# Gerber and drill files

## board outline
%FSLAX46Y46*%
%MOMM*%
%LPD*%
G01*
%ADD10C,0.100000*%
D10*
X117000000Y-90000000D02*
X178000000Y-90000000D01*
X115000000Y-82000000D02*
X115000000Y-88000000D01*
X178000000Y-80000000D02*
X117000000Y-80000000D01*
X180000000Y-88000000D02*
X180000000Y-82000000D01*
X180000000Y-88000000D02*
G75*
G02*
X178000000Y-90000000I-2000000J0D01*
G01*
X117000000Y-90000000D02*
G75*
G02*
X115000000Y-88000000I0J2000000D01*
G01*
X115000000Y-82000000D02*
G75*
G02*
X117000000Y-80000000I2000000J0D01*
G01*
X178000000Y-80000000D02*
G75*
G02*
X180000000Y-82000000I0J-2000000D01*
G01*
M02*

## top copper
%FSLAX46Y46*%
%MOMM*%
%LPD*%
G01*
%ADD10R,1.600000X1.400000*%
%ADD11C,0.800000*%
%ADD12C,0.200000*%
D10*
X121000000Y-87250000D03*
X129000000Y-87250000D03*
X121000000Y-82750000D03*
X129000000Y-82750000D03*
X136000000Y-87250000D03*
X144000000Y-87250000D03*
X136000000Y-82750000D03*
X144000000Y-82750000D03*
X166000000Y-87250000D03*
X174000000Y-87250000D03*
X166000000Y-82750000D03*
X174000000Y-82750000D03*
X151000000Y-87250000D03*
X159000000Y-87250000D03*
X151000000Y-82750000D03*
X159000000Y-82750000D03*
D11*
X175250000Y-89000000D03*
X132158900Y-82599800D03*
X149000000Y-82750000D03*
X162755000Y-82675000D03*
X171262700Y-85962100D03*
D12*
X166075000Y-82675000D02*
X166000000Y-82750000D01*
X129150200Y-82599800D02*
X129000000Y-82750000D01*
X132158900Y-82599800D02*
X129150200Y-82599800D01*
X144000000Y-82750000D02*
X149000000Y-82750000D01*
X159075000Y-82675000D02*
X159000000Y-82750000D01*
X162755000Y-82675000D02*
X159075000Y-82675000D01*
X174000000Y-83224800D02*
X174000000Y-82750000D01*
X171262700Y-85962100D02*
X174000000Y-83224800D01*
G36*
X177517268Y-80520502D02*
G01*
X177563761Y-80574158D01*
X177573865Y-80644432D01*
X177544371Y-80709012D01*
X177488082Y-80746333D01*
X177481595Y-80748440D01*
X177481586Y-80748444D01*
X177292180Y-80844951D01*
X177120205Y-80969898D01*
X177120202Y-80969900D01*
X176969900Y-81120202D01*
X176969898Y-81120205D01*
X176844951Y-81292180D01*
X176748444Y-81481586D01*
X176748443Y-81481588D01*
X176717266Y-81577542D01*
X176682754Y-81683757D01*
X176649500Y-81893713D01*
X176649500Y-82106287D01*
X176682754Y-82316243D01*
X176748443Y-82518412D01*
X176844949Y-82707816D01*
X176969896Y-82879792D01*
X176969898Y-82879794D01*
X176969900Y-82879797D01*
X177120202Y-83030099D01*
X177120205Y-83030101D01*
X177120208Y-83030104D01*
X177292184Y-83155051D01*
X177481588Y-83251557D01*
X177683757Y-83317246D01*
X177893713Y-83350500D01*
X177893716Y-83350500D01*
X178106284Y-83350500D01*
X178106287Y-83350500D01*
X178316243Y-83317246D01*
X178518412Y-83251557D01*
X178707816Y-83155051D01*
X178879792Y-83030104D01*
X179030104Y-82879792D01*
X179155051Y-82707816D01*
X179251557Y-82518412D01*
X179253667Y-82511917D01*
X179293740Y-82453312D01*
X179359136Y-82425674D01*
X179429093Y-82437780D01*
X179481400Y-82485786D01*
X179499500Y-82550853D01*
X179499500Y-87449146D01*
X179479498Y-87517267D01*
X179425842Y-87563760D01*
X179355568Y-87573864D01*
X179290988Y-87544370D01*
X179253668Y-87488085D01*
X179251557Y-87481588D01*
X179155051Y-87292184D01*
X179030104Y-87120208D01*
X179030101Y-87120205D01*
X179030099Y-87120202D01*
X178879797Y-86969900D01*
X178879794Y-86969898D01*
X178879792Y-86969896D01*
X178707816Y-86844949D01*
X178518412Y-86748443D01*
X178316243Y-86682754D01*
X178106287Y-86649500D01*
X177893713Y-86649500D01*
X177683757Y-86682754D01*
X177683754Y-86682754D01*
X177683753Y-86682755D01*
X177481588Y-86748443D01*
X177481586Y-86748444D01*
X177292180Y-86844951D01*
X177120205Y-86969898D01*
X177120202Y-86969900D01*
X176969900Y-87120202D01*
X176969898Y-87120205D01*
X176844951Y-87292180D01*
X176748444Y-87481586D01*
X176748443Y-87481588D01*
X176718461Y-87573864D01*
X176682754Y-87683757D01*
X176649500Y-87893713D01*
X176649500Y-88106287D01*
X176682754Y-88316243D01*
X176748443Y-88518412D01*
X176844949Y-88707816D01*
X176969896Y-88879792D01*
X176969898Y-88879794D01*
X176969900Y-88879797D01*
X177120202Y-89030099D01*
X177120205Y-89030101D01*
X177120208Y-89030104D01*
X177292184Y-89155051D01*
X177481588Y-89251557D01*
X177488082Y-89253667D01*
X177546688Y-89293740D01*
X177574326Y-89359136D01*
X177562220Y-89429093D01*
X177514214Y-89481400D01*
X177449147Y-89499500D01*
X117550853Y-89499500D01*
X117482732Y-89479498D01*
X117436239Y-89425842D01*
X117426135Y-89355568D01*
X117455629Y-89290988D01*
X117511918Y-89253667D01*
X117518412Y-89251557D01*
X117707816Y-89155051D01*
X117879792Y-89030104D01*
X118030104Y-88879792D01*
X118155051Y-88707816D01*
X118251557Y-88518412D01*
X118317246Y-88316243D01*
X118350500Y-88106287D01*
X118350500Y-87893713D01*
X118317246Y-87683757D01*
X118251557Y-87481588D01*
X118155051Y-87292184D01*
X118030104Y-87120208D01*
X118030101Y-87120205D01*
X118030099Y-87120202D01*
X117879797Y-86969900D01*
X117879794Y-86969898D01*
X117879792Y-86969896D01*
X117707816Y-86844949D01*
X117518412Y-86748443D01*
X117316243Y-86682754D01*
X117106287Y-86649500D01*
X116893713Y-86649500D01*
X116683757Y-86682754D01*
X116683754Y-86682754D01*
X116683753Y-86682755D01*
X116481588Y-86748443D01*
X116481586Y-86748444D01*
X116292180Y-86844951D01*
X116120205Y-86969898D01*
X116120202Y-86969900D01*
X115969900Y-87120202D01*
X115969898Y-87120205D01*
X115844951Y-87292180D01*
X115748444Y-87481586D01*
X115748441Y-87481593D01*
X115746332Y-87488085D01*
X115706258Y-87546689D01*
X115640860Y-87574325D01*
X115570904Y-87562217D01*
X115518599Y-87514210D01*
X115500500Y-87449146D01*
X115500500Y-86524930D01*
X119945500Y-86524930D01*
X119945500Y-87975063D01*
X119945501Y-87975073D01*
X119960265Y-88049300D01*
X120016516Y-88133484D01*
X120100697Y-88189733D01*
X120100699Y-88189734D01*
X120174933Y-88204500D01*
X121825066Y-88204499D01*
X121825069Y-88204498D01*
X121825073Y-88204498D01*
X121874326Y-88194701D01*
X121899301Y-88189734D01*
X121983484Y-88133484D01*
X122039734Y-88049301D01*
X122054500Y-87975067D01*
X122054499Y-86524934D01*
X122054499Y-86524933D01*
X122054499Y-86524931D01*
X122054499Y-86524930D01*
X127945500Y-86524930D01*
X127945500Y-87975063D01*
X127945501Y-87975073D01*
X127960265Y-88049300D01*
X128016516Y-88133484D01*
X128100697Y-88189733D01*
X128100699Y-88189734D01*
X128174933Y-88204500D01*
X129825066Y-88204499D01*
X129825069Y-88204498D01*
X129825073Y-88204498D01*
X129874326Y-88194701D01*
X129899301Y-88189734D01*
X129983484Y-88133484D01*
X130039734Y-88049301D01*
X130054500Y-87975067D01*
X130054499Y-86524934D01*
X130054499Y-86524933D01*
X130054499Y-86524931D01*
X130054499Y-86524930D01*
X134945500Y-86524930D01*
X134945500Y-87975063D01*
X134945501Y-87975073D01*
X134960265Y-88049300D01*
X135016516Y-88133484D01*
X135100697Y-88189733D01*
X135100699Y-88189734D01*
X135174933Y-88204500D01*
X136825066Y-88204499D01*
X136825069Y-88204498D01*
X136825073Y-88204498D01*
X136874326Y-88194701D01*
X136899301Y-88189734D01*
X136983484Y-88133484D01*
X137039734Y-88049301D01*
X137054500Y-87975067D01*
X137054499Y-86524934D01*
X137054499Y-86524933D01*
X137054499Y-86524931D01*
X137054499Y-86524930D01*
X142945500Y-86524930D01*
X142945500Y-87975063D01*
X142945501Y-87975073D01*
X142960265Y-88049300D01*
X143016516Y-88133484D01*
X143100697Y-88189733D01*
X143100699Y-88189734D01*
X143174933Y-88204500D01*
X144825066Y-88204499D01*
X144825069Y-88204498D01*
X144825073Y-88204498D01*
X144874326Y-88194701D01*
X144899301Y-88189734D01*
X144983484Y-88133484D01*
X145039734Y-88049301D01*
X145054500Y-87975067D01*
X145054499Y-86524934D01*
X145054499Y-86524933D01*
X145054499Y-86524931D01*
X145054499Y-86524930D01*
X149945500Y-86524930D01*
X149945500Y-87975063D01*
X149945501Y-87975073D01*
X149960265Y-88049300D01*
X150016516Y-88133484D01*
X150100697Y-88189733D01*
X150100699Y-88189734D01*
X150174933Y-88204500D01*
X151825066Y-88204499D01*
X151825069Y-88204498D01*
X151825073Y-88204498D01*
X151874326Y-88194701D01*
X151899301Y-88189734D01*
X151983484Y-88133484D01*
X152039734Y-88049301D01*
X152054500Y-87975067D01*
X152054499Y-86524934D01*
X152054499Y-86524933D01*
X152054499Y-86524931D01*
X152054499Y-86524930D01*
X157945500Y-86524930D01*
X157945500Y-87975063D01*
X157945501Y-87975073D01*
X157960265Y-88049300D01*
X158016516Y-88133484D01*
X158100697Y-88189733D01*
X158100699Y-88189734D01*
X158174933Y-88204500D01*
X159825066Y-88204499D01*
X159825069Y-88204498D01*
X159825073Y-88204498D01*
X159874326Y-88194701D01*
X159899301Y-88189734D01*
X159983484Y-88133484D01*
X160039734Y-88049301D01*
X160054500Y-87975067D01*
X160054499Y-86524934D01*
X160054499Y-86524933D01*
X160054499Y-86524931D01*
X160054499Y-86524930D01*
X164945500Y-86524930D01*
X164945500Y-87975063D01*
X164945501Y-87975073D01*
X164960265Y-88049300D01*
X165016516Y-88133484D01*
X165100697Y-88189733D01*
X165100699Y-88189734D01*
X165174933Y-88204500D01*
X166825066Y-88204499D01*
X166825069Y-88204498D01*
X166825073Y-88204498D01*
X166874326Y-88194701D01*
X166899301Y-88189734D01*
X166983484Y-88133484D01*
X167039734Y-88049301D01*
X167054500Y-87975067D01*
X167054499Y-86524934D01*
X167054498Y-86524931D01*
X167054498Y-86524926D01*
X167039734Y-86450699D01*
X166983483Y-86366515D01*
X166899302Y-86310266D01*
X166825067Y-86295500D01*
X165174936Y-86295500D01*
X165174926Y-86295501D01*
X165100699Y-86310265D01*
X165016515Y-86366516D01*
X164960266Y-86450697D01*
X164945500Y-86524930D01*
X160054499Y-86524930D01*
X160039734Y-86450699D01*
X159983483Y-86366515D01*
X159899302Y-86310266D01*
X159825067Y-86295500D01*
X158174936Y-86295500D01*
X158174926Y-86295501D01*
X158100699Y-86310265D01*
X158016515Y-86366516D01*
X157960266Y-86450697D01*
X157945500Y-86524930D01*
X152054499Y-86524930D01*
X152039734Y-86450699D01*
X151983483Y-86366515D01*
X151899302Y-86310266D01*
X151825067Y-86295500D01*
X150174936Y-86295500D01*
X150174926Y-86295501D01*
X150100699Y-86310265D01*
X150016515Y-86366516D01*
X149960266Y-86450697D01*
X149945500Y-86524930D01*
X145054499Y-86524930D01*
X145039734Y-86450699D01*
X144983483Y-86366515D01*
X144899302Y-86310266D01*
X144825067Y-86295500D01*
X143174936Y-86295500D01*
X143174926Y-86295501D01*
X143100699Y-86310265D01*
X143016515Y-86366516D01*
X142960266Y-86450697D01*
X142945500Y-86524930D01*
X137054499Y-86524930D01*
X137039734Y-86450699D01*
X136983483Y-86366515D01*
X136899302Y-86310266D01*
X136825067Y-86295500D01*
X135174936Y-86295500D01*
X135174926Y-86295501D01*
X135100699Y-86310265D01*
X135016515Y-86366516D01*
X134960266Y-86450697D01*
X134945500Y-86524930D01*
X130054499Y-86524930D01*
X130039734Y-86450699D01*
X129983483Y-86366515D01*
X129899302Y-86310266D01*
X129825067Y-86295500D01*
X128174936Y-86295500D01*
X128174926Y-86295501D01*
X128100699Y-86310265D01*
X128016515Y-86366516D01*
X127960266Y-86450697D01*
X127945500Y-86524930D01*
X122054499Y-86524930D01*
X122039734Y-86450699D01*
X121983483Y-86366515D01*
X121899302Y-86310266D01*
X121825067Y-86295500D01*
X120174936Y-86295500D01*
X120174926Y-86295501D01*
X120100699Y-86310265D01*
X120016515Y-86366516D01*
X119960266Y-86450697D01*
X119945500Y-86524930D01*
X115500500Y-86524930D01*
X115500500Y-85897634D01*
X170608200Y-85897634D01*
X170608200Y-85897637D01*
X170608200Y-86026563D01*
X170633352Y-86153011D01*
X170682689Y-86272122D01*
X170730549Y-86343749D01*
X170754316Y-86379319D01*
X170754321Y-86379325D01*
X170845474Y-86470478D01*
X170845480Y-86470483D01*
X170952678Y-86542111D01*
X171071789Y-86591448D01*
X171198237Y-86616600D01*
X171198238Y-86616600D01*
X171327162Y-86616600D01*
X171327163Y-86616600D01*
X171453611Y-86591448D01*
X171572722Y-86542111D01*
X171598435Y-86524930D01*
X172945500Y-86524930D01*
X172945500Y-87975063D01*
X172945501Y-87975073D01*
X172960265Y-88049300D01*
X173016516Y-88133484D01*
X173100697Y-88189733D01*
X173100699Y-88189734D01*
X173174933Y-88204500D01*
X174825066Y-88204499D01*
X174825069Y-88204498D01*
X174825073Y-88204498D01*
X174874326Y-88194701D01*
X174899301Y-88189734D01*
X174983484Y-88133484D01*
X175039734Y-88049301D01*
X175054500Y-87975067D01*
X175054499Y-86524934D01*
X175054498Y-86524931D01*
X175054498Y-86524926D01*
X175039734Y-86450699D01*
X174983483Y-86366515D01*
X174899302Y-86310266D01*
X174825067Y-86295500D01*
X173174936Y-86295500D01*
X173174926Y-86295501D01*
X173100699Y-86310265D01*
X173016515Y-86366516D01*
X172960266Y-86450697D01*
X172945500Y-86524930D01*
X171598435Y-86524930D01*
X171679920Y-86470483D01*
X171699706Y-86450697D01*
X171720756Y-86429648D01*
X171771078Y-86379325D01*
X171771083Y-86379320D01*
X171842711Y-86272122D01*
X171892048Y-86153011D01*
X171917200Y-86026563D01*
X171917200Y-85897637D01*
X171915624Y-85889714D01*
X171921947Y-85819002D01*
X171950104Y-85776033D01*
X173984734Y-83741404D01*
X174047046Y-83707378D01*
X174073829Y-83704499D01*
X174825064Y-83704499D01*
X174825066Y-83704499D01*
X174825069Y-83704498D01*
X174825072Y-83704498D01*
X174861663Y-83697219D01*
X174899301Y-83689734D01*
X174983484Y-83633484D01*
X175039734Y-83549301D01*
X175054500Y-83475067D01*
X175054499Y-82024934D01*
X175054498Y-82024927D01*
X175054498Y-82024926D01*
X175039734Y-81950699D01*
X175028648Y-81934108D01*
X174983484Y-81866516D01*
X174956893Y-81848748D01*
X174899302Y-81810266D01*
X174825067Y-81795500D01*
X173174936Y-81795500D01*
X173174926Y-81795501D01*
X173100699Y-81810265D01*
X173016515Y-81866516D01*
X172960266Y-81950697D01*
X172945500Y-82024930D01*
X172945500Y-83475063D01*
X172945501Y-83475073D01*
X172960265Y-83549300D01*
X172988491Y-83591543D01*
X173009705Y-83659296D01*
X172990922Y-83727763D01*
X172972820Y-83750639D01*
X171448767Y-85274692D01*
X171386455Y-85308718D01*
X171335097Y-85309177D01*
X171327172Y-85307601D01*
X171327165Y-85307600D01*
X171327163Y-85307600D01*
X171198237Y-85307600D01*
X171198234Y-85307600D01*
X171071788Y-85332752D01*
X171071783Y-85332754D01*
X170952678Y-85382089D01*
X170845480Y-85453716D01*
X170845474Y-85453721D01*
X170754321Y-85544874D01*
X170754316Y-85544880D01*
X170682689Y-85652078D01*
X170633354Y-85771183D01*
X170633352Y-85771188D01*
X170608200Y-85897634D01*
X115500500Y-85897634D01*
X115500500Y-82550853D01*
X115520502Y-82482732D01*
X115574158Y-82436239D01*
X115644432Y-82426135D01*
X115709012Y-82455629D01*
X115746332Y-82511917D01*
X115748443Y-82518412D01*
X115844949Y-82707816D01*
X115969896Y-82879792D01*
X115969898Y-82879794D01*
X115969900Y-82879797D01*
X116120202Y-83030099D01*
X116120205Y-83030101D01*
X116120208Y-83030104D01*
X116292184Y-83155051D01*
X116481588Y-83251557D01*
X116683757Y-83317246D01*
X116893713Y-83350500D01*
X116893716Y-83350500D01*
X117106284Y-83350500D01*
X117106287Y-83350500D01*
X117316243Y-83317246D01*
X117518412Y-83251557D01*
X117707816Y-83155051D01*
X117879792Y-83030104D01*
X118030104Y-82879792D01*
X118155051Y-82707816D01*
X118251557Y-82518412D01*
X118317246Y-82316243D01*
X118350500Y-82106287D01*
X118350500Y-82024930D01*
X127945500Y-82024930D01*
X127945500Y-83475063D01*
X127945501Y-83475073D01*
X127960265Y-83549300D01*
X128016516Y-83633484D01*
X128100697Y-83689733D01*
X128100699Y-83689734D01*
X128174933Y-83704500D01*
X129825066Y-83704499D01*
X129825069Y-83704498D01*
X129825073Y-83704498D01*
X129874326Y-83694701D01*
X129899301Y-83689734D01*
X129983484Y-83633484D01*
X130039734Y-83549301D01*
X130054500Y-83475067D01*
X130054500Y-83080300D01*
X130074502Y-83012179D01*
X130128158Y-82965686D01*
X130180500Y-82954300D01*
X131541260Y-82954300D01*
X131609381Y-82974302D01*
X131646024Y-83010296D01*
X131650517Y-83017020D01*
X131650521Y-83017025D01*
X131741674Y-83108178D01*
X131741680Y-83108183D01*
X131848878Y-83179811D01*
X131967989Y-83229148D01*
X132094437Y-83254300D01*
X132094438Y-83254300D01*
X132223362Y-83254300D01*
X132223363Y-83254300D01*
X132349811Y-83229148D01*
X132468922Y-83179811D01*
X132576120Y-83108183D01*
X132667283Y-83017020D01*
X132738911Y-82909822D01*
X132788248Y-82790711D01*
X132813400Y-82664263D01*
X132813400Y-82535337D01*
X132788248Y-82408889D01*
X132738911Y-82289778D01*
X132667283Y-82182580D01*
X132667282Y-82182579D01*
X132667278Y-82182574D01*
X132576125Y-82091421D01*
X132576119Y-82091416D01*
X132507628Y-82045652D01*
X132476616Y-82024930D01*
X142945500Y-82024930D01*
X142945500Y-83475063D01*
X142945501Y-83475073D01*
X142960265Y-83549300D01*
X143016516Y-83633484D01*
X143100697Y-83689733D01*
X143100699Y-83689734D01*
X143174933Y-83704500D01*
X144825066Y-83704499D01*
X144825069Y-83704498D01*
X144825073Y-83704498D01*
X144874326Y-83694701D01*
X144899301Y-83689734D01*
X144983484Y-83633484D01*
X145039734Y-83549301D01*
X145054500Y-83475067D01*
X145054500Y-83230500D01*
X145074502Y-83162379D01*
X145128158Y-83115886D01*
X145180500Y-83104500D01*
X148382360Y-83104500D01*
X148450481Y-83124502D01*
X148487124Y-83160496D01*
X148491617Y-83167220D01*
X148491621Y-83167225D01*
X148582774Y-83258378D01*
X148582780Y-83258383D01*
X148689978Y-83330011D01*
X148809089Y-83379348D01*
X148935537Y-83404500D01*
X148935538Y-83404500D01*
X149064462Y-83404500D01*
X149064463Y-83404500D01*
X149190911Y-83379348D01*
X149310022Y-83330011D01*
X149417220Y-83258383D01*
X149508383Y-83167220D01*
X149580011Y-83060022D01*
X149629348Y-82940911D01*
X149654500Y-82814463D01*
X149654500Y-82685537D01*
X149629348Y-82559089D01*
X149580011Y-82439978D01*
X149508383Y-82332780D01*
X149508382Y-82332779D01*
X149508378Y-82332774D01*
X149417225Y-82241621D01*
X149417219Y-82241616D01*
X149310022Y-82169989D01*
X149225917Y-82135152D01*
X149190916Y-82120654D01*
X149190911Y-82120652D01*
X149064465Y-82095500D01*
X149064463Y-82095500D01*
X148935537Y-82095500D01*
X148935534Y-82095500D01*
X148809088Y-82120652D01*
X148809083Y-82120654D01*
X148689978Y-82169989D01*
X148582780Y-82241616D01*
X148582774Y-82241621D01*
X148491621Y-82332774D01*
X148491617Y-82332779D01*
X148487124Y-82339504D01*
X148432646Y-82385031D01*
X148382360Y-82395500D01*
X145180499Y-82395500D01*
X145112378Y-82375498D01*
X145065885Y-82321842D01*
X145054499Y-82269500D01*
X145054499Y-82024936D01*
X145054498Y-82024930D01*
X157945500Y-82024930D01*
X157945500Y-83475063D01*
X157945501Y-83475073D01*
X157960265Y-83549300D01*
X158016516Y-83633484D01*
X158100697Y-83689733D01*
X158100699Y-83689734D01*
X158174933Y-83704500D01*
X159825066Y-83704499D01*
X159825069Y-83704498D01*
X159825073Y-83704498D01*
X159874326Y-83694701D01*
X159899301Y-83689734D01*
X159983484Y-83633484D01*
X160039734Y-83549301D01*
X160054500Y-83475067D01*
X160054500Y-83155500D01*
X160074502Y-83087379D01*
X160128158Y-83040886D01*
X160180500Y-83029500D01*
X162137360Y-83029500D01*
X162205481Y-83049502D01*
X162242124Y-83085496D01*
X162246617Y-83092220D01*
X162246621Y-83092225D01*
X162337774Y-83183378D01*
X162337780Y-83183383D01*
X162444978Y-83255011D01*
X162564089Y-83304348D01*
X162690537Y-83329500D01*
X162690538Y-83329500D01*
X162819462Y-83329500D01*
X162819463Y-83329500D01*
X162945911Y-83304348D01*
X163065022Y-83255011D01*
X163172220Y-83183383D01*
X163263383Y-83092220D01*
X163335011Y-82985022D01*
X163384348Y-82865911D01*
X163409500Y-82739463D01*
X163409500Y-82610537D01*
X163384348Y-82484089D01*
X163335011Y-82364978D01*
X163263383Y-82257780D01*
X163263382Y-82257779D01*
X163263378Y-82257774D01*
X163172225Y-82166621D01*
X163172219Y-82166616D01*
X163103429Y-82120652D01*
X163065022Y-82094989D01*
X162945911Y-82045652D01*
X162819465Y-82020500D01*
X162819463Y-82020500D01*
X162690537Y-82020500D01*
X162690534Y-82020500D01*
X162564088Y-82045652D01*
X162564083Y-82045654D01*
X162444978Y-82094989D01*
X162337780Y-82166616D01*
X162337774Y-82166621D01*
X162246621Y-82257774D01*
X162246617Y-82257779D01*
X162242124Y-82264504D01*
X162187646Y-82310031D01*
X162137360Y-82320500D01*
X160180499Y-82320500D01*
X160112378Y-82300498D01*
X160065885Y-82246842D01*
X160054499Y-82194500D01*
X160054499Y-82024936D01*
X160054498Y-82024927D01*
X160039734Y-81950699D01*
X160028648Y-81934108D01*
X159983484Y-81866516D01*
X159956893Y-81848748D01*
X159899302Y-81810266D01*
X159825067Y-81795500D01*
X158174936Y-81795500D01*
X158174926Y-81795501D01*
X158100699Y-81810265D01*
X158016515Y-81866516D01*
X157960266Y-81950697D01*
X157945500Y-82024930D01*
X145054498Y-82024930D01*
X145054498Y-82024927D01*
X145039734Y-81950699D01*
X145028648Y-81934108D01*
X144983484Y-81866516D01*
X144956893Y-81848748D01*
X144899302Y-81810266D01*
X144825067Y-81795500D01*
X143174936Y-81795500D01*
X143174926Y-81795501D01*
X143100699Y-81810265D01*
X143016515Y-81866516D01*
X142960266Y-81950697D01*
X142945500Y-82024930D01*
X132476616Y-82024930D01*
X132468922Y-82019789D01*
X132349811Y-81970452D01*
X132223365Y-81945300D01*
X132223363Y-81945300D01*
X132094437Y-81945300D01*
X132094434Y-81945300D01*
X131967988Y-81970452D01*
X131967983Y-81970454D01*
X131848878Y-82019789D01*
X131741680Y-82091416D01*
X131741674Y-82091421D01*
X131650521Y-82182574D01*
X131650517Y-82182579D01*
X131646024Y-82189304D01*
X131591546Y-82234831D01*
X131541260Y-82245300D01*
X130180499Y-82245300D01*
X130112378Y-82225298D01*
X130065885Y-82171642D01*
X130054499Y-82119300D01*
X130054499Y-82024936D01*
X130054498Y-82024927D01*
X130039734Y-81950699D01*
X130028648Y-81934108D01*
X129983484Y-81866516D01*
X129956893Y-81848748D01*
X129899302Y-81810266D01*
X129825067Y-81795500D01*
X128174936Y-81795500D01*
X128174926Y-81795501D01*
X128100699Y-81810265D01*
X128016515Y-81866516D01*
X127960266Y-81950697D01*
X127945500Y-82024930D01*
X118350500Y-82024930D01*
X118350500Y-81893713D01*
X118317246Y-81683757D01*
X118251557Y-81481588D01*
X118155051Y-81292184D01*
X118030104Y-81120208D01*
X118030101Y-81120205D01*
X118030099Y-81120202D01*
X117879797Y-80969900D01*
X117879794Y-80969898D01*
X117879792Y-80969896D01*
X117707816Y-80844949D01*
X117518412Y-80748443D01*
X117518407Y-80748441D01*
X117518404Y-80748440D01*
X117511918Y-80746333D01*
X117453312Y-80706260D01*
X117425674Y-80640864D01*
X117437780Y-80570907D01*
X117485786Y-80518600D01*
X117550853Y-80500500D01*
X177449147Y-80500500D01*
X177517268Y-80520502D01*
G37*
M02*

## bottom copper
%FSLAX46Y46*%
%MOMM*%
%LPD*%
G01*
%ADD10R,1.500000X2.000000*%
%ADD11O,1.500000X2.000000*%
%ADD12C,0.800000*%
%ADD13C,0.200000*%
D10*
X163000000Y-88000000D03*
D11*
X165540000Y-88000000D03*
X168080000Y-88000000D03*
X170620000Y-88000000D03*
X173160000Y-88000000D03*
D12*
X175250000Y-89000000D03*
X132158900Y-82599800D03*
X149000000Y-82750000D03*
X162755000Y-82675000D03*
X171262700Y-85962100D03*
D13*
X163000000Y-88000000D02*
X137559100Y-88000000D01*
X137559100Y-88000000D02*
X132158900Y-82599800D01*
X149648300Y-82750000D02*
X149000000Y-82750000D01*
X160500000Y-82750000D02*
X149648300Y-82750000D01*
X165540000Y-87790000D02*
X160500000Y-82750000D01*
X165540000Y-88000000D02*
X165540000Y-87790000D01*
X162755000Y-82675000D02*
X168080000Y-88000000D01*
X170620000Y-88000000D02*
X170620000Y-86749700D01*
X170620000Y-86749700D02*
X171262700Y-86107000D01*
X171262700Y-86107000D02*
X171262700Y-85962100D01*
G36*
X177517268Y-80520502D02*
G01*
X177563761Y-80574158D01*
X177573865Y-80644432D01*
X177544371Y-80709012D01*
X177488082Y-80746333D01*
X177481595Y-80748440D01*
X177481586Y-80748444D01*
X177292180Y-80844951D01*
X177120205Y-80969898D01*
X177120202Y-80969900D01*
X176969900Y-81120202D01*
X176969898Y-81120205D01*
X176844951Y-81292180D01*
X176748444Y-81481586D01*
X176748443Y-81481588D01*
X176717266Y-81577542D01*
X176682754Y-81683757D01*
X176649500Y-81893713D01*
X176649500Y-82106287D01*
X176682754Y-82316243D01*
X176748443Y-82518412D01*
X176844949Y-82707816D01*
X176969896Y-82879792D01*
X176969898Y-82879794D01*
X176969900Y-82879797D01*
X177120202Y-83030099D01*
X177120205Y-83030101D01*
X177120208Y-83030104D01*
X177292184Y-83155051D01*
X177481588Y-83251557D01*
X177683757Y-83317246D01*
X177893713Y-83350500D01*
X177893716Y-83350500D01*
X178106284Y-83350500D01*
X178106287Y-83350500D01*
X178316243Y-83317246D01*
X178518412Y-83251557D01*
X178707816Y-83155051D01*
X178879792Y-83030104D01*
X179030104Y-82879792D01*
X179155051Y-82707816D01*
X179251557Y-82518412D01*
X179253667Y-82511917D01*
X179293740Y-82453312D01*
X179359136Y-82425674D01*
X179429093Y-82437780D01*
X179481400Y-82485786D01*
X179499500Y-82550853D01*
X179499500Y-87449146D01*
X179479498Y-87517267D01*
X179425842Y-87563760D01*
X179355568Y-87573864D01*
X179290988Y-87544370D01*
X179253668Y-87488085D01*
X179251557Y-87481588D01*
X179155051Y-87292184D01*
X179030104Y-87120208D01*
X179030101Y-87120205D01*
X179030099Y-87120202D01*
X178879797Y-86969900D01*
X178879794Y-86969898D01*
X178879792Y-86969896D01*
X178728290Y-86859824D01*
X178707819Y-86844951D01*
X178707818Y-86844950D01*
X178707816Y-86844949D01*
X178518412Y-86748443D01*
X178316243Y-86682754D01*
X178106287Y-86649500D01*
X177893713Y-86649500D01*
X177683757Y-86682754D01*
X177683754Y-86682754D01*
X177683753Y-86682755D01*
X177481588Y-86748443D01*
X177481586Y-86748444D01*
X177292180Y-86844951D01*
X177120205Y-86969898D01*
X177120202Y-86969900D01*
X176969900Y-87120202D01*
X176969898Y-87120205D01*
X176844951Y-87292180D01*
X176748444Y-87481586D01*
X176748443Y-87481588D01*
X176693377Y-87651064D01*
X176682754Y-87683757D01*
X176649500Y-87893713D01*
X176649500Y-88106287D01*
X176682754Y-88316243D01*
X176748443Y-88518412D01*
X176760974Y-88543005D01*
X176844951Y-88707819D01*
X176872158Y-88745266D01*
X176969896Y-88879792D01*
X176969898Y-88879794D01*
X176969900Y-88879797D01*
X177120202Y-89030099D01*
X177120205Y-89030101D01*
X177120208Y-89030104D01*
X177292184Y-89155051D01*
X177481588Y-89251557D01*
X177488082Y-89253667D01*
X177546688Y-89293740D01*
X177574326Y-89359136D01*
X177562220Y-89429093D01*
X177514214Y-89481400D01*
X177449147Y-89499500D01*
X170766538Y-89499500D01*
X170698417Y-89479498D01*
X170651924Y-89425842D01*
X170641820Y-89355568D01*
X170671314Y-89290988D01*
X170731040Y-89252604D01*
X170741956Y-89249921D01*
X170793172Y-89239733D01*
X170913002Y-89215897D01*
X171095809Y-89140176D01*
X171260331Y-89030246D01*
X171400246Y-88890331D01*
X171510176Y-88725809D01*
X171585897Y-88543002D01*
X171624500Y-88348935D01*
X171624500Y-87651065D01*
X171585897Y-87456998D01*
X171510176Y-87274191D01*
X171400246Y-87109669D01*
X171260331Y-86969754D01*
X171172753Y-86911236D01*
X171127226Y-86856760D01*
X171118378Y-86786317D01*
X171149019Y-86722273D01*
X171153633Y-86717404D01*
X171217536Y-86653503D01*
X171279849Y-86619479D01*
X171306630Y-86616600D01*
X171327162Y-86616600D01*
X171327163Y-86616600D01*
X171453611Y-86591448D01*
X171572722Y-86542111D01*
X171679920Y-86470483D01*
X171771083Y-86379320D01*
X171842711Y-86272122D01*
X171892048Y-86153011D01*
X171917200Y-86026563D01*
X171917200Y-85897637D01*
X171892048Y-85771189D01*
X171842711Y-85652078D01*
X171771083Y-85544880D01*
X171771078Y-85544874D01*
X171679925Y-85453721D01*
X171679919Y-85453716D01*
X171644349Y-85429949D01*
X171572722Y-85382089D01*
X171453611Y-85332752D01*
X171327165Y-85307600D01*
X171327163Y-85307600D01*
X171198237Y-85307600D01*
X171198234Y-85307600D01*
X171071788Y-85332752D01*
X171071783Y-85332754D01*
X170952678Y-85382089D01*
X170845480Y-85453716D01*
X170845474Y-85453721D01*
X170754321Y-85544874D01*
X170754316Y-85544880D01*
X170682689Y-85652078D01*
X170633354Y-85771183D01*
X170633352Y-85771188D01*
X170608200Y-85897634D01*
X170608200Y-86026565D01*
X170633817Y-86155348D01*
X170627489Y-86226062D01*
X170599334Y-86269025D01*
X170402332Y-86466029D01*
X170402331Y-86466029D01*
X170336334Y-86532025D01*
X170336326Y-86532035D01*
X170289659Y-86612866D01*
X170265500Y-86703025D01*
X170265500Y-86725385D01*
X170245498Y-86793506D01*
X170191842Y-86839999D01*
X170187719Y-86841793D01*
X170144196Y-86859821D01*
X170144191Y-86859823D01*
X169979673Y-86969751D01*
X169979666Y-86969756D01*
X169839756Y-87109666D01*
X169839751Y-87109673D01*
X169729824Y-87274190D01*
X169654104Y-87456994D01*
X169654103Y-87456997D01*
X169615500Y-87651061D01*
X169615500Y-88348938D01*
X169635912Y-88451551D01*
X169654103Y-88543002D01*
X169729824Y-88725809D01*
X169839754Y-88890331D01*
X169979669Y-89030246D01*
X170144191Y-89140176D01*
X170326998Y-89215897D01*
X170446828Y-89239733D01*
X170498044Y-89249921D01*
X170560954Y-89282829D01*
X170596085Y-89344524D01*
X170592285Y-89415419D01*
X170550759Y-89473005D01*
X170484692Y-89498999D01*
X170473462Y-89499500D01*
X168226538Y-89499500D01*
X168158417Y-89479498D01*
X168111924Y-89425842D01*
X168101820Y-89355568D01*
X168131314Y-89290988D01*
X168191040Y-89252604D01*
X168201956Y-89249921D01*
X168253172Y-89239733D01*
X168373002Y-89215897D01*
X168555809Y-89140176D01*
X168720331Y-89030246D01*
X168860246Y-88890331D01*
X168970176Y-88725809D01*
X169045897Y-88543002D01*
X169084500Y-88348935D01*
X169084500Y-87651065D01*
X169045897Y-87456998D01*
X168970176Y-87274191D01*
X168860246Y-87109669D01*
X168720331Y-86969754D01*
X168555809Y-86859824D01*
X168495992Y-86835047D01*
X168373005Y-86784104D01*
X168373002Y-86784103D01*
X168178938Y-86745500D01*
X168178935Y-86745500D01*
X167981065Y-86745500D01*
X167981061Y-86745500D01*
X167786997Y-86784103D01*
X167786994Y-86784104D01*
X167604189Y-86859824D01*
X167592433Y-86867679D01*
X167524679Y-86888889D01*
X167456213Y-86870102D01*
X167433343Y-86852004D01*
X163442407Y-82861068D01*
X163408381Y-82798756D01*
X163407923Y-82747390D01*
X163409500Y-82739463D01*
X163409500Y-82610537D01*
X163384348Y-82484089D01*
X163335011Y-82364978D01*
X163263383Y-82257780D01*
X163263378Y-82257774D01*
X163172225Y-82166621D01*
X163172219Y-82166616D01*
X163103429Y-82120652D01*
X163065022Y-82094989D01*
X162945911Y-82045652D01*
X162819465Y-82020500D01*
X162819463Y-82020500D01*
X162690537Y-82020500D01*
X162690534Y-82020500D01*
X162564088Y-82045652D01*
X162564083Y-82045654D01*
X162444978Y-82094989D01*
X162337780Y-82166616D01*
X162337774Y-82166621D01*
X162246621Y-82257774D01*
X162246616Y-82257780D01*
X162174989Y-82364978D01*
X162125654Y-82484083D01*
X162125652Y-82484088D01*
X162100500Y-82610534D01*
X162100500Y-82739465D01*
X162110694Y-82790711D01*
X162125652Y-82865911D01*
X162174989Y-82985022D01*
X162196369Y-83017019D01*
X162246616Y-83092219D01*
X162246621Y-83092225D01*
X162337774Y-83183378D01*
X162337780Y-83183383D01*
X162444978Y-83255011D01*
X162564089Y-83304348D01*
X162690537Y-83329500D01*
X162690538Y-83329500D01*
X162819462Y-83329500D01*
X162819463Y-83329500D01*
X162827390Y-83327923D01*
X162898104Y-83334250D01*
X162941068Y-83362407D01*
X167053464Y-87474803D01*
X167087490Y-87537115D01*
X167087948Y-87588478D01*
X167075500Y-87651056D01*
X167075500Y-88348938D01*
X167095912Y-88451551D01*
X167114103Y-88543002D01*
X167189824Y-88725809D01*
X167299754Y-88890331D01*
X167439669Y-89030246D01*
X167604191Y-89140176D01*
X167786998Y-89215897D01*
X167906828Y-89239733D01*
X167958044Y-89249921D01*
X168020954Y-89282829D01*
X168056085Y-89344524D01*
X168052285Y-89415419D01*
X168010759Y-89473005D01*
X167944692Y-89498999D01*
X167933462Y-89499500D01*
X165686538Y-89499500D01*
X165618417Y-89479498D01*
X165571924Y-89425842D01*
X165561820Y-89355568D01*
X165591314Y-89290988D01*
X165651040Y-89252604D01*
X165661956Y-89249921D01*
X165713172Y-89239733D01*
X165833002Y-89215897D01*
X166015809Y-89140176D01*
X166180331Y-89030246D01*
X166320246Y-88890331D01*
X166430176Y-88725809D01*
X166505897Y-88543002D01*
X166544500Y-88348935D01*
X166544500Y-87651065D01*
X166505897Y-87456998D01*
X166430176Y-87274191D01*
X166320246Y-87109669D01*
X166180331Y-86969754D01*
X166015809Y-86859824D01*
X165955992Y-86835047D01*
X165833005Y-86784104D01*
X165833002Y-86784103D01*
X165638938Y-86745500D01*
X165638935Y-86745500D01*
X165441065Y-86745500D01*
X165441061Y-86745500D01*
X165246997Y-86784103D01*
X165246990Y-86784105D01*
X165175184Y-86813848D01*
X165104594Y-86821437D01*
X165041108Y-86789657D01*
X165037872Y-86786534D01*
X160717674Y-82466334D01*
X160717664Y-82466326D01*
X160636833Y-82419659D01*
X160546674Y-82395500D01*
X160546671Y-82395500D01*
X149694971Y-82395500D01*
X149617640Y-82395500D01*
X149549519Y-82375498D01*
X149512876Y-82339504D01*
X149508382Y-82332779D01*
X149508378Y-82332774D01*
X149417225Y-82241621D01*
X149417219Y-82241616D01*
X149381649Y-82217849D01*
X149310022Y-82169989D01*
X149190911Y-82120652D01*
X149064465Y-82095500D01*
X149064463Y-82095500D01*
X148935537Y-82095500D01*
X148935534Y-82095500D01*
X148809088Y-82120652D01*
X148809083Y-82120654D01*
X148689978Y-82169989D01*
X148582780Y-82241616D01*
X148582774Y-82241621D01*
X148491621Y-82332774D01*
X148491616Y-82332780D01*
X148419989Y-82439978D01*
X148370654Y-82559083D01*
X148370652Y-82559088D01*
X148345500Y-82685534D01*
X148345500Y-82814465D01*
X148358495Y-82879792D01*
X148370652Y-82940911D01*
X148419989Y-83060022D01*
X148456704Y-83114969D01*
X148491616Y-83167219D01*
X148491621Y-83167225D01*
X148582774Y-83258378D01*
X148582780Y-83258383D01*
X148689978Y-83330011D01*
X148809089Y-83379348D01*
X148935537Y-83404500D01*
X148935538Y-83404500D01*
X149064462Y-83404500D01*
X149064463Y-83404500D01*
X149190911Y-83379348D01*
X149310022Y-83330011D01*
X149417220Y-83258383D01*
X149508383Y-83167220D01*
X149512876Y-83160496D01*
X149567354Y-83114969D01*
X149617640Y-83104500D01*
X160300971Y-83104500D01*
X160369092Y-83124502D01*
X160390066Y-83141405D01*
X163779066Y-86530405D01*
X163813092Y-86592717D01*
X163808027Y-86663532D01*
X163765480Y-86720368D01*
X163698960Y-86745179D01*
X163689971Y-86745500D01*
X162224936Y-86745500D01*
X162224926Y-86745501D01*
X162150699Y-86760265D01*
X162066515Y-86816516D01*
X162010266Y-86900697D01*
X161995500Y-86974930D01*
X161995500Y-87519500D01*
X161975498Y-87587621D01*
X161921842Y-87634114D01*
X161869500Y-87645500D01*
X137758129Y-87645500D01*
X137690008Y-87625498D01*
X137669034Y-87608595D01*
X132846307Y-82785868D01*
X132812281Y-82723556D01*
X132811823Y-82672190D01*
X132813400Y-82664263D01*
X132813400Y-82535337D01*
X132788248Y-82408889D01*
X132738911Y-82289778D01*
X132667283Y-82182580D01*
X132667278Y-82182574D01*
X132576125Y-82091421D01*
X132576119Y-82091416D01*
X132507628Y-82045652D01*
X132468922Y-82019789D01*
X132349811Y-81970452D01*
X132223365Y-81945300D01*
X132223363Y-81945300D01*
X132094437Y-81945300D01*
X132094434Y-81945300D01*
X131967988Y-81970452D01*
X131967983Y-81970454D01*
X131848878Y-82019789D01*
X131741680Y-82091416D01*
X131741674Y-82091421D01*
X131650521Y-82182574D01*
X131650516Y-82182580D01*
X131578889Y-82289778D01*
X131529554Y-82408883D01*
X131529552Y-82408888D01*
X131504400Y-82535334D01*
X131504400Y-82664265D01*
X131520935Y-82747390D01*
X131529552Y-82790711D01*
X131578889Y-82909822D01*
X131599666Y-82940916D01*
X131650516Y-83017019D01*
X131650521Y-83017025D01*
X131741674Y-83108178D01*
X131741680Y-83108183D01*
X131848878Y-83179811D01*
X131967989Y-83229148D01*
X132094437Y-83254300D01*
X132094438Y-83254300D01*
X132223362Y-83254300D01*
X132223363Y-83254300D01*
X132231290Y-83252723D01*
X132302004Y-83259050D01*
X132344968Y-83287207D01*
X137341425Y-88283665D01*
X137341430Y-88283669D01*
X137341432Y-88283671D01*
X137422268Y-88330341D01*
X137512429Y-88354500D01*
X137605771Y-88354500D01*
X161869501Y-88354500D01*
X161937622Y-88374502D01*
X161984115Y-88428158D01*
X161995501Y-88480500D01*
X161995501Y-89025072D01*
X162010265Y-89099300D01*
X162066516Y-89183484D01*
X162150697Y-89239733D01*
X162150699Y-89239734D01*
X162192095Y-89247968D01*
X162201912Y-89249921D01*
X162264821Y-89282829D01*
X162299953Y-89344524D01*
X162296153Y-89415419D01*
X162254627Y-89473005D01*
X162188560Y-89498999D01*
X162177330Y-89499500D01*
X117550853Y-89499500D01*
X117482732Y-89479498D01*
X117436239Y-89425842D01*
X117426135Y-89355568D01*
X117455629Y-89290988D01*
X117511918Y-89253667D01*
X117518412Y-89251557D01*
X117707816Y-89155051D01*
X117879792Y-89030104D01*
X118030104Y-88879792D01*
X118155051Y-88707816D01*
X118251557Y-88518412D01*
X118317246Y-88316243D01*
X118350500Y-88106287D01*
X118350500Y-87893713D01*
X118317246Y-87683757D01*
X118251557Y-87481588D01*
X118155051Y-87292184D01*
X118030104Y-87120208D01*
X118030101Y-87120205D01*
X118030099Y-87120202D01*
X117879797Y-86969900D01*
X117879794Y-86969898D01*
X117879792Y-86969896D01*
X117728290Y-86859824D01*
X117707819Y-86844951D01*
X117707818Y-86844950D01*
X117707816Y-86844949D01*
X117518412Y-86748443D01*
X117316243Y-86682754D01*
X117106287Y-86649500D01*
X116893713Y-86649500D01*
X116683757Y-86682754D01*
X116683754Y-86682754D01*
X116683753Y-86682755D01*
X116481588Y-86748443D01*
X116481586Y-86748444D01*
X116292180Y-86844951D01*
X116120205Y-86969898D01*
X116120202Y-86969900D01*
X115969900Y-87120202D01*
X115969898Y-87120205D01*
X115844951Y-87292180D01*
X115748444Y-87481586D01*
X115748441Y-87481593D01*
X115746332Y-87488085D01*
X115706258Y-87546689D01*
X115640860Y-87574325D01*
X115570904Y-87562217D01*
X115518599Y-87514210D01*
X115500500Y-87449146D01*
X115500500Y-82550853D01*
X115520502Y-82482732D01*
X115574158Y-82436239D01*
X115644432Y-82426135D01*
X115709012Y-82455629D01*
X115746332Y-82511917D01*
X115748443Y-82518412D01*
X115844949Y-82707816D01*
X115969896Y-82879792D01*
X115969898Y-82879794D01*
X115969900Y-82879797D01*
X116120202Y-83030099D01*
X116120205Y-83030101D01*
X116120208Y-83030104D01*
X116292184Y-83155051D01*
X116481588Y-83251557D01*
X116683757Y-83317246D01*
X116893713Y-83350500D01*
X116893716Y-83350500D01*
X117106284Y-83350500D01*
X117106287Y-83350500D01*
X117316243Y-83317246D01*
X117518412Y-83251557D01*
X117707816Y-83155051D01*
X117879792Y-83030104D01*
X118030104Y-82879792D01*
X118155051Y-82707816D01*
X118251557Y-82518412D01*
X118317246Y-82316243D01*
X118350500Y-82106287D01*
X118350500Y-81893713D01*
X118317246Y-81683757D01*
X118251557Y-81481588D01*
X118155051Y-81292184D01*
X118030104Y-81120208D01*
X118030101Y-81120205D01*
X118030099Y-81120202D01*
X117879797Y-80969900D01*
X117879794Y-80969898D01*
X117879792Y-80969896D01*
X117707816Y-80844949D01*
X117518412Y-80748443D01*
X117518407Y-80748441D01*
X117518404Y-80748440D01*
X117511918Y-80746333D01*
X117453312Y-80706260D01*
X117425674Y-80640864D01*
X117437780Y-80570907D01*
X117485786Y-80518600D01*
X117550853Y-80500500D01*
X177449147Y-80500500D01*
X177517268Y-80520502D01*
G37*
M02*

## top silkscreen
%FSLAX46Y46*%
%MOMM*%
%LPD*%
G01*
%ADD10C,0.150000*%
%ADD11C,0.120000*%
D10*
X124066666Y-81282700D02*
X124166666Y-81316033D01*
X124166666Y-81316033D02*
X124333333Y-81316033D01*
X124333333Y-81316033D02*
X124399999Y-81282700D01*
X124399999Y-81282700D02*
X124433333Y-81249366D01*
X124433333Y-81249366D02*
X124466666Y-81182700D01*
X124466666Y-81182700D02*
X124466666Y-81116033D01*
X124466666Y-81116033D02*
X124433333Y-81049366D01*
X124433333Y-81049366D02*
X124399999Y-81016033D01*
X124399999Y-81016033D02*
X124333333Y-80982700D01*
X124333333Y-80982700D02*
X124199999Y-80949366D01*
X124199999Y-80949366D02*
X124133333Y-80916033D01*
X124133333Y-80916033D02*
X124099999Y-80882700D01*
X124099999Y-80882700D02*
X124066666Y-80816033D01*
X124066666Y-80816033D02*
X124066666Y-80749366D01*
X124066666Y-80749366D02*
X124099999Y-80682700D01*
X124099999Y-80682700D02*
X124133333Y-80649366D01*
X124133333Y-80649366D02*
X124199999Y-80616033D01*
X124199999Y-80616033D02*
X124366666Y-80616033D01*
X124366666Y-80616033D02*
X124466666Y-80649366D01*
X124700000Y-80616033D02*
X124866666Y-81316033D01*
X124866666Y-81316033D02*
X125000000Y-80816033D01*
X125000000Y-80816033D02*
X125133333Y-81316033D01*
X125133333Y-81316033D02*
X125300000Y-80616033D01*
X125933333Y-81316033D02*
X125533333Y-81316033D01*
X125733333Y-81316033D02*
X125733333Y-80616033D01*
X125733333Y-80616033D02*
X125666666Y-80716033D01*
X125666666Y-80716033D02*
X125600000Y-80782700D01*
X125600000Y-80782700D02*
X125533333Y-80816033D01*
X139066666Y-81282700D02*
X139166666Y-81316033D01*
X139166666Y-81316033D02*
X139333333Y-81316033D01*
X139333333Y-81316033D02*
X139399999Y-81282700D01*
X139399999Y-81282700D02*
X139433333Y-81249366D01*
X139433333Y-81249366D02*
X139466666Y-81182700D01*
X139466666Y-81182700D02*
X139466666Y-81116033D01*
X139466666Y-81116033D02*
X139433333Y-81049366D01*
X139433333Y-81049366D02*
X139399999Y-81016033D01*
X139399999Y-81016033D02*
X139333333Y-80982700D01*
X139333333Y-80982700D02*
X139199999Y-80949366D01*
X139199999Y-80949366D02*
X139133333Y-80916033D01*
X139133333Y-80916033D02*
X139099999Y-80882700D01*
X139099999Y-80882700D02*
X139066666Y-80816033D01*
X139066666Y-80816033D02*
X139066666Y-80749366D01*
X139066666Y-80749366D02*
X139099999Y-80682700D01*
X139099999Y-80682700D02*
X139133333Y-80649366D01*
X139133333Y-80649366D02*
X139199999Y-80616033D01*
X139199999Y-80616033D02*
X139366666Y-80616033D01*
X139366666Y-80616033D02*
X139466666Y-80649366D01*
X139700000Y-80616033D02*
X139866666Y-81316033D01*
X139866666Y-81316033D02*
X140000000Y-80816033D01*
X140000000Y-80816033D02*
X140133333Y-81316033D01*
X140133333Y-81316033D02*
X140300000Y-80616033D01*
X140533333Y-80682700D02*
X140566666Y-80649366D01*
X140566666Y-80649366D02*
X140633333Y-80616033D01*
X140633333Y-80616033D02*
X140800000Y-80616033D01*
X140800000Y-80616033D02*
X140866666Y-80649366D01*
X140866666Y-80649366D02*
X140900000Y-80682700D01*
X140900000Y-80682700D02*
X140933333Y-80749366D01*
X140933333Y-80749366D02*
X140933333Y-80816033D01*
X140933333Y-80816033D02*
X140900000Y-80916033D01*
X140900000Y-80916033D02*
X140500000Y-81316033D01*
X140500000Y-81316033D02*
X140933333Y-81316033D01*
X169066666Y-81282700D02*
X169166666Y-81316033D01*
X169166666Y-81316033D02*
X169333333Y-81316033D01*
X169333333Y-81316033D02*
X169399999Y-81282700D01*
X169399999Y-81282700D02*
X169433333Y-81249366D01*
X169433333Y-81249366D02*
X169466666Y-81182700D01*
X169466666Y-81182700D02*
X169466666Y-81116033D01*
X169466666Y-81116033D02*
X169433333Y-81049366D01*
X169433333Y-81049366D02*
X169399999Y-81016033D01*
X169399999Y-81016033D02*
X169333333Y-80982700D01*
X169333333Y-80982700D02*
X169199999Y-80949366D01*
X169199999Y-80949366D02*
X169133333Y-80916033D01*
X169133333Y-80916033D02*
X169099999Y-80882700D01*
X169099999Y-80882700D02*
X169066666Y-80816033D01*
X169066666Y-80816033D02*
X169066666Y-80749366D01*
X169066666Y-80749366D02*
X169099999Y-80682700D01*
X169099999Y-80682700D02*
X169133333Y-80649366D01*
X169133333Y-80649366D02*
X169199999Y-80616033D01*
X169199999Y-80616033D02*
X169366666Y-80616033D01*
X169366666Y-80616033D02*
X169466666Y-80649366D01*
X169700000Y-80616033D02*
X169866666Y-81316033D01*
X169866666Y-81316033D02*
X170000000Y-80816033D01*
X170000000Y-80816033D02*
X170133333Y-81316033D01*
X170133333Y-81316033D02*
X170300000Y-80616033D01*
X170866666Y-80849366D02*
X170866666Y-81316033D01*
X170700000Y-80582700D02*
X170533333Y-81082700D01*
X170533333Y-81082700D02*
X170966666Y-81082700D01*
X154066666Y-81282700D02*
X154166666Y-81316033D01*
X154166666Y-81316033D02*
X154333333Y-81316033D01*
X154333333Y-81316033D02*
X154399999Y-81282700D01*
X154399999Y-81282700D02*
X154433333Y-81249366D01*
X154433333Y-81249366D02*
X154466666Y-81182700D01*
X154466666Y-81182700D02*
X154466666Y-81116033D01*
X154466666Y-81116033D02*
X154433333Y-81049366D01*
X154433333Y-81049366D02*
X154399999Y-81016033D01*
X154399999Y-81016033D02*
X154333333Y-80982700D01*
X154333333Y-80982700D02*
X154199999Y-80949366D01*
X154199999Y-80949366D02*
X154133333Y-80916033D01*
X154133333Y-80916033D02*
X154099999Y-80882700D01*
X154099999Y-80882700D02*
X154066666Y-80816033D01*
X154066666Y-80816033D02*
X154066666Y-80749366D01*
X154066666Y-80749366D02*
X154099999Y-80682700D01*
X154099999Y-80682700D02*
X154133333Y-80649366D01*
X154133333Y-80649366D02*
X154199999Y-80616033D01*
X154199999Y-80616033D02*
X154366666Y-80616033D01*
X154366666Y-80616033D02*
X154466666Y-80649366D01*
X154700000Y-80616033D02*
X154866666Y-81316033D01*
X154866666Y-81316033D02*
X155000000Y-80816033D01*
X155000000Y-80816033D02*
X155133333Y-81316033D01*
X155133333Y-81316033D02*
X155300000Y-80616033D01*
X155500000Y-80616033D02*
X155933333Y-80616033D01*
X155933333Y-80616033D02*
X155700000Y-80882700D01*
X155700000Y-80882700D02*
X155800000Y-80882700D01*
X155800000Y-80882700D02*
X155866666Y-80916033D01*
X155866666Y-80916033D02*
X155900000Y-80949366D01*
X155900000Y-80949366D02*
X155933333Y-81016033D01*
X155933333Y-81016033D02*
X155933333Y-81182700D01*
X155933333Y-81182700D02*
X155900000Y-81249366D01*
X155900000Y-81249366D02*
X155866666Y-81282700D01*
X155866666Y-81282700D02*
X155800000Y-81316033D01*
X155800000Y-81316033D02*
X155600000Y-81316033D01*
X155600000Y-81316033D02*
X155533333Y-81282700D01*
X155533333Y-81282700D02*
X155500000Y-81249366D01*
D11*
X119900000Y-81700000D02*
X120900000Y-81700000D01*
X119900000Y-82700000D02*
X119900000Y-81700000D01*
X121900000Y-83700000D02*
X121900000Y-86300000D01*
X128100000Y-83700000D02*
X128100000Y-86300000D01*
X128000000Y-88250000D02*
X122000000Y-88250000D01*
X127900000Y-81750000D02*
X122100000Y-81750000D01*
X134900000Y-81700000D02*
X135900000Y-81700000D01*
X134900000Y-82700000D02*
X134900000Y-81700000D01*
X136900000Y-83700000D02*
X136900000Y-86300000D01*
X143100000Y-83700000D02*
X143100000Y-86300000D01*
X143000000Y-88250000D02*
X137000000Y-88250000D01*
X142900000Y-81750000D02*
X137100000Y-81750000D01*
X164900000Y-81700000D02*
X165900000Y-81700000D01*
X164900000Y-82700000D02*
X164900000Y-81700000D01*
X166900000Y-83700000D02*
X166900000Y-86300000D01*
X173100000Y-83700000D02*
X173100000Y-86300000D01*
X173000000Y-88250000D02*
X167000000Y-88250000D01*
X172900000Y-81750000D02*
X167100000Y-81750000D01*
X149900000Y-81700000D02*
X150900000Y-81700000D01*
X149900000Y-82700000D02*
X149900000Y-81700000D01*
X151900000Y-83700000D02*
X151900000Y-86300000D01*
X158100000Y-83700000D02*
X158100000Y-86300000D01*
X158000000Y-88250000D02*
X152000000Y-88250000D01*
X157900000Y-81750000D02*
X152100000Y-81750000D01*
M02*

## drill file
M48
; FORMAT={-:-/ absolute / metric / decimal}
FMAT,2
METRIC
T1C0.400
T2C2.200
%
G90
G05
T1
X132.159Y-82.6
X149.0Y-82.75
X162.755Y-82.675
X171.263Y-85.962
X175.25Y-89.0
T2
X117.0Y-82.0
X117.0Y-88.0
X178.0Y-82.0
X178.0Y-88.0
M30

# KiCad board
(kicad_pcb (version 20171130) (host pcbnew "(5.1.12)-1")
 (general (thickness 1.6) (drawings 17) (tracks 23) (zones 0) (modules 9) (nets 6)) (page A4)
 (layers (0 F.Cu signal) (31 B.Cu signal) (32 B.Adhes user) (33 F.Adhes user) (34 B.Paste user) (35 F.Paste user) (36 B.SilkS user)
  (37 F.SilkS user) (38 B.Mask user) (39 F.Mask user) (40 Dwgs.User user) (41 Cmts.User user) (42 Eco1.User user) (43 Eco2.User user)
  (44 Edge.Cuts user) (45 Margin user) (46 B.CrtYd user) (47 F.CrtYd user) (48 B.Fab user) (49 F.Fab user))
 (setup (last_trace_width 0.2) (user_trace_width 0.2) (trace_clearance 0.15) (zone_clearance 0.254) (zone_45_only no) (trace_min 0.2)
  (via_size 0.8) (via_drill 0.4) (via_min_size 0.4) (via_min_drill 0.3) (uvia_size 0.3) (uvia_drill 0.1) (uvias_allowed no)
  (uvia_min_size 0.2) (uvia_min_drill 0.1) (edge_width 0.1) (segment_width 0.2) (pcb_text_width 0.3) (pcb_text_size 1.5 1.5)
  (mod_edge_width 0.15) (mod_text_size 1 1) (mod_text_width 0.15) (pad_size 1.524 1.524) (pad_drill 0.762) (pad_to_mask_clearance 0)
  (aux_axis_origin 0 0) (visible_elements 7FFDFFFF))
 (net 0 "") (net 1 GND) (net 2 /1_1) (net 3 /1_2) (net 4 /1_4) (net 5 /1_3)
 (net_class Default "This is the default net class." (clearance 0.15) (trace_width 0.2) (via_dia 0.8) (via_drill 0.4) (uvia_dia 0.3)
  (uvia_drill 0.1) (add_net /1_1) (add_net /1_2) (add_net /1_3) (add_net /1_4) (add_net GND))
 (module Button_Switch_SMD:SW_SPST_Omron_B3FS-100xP (layer F.Cu) (at 125 85)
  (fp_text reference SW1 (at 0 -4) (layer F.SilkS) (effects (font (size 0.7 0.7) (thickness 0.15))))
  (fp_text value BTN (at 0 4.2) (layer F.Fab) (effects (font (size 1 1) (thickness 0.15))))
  (fp_line (start -5.1 -3.3) (end -4.1 -3.3) (layer F.SilkS) (width 0.12))
  (fp_line (start -5.1 -2.3) (end -5.1 -3.3) (layer F.SilkS) (width 0.12))
  (fp_line (start -3.1 -1.3) (end -3.1 1.3) (layer F.SilkS) (width 0.12))
  (fp_line (start 3.1 -1.3) (end 3.1 1.3) (layer F.SilkS) (width 0.12))
  (fp_line (start 3 3.25) (end -3 3.25) (layer F.SilkS) (width 0.12))
  (fp_line (start 2.9 -3.25) (end -2.9 -3.25) (layer F.SilkS) (width 0.12))
  (pad 3 smd rect (at -4 2.25 180) (size 1.6 1.4) (layers F.Cu F.Paste F.Mask))
  (pad 4 smd rect (at 4 2.25 180) (size 1.6 1.4) (layers F.Cu F.Paste F.Mask))
  (pad 1 smd rect (at -4 -2.25 180) (size 1.6 1.4) (layers F.Cu F.Paste F.Mask) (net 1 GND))
  (pad 2 smd rect (at 4 -2.25 180) (size 1.6 1.4) (layers F.Cu F.Paste F.Mask) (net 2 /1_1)))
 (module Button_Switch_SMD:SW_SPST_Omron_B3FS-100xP (layer F.Cu) (at 140 85)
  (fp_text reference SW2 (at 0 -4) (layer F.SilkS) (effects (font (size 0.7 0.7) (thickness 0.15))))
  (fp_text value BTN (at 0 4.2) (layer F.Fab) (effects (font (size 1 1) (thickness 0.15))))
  (fp_line (start -5.1 -3.3) (end -4.1 -3.3) (layer F.SilkS) (width 0.12))
  (fp_line (start -5.1 -2.3) (end -5.1 -3.3) (layer F.SilkS) (width 0.12))
  (fp_line (start -3.1 -1.3) (end -3.1 1.3) (layer F.SilkS) (width 0.12))
  (fp_line (start 3.1 -1.3) (end 3.1 1.3) (layer F.SilkS) (width 0.12))
  (fp_line (start 3 3.25) (end -3 3.25) (layer F.SilkS) (width 0.12))
  (fp_line (start 2.9 -3.25) (end -2.9 -3.25) (layer F.SilkS) (width 0.12))
  (pad 3 smd rect (at -4 2.25 180) (size 1.6 1.4) (layers F.Cu F.Paste F.Mask))
  (pad 4 smd rect (at 4 2.25 180) (size 1.6 1.4) (layers F.Cu F.Paste F.Mask))
  (pad 1 smd rect (at -4 -2.25 180) (size 1.6 1.4) (layers F.Cu F.Paste F.Mask) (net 1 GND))
  (pad 2 smd rect (at 4 -2.25 180) (size 1.6 1.4) (layers F.Cu F.Paste F.Mask) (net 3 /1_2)))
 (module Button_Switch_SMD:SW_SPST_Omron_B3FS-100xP (layer F.Cu) (at 170 85)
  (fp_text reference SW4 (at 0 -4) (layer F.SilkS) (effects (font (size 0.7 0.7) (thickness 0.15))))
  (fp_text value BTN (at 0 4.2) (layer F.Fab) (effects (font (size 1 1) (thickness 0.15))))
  (fp_line (start -5.1 -3.3) (end -4.1 -3.3) (layer F.SilkS) (width 0.12))
  (fp_line (start -5.1 -2.3) (end -5.1 -3.3) (layer F.SilkS) (width 0.12))
  (fp_line (start -3.1 -1.3) (end -3.1 1.3) (layer F.SilkS) (width 0.12))
  (fp_line (start 3.1 -1.3) (end 3.1 1.3) (layer F.SilkS) (width 0.12))
  (fp_line (start 3 3.25) (end -3 3.25) (layer F.SilkS) (width 0.12))
  (fp_line (start 2.9 -3.25) (end -2.9 -3.25) (layer F.SilkS) (width 0.12))
  (pad 3 smd rect (at -4 2.25 180) (size 1.6 1.4) (layers F.Cu F.Paste F.Mask))
  (pad 4 smd rect (at 4 2.25 180) (size 1.6 1.4) (layers F.Cu F.Paste F.Mask))
  (pad 1 smd rect (at -4 -2.25 180) (size 1.6 1.4) (layers F.Cu F.Paste F.Mask) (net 1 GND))
  (pad 2 smd rect (at 4 -2.25 180) (size 1.6 1.4) (layers F.Cu F.Paste F.Mask) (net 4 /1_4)))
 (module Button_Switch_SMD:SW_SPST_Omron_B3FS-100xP (layer F.Cu) (at 155 85)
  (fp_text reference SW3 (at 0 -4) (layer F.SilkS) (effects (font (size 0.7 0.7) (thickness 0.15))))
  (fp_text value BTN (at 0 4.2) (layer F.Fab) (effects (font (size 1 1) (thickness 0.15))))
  (fp_line (start -5.1 -3.3) (end -4.1 -3.3) (layer F.SilkS) (width 0.12))
  (fp_line (start -5.1 -2.3) (end -5.1 -3.3) (layer F.SilkS) (width 0.12))
  (fp_line (start -3.1 -1.3) (end -3.1 1.3) (layer F.SilkS) (width 0.12))
  (fp_line (start 3.1 -1.3) (end 3.1 1.3) (layer F.SilkS) (width 0.12))
  (fp_line (start 3 3.25) (end -3 3.25) (layer F.SilkS) (width 0.12))
  (fp_line (start 2.9 -3.25) (end -2.9 -3.25) (layer F.SilkS) (width 0.12))
  (pad 3 smd rect (at -4 2.25 180) (size 1.6 1.4) (layers F.Cu F.Paste F.Mask))
  (pad 4 smd rect (at 4 2.25 180) (size 1.6 1.4) (layers F.Cu F.Paste F.Mask))
  (pad 1 smd rect (at -4 -2.25 180) (size 1.6 1.4) (layers F.Cu F.Paste F.Mask) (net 1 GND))
  (pad 2 smd rect (at 4 -2.25 180) (size 1.6 1.4) (layers F.Cu F.Paste F.Mask) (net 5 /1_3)))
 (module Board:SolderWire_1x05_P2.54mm (layer B.Cu) (at 163 88 270)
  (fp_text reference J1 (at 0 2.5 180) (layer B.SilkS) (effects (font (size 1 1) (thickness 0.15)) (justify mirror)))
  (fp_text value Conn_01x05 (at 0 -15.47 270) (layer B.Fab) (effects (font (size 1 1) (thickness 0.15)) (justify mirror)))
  (pad 1 smd rect (at 0 0 270) (size 2 1.5) (layers B.Cu B.Paste B.Mask) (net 2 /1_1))
  (pad 2 smd oval (at 0 -2.54 270) (size 2 1.5) (layers B.Cu B.Paste B.Mask) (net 3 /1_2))
  (pad 3 smd oval (at 0 -5.08 270) (size 2 1.5) (layers B.Cu B.Paste B.Mask) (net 5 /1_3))
  (pad 4 smd oval (at 0 -7.62 270) (size 2 1.5) (layers B.Cu B.Paste B.Mask) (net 4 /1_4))
  (pad 5 smd oval (at 0 -10.16 270) (size 2 1.5) (layers B.Cu B.Paste B.Mask) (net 1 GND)))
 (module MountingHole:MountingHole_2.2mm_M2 (layer F.Cu) (at 117 88)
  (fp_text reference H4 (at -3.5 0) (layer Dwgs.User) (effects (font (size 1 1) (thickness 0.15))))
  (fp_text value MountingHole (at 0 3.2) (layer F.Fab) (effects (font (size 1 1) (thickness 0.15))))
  (pad 1 np_thru_hole circle (at 0 0) (size 2.2 2.2) (drill 2.2) (layers *.Cu *.Mask)))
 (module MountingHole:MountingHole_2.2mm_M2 (layer F.Cu) (at 178 88)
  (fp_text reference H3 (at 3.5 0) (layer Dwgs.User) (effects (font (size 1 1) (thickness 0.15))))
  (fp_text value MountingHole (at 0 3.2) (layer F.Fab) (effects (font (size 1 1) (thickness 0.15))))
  (pad 1 np_thru_hole circle (at 0 0) (size 2.2 2.2) (drill 2.2) (layers *.Cu *.Mask)))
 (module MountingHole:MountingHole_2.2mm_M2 (layer F.Cu) (at 178 82)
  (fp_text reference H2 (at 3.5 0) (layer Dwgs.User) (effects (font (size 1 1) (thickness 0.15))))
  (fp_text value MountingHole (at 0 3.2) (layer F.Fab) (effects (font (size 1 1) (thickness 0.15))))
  (pad 1 np_thru_hole circle (at 0 0) (size 2.2 2.2) (drill 2.2) (layers *.Cu *.Mask)))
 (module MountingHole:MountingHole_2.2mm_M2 (layer F.Cu) (at 117 82)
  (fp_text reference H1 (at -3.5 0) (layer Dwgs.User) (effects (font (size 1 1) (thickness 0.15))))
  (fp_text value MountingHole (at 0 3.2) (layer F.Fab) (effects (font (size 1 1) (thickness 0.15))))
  (pad 1 np_thru_hole circle (at 0 0) (size 2.2 2.2) (drill 2.2) (layers *.Cu *.Mask)))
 (gr_line (start 117 90) (end 178 90) (layer Edge.Cuts) (width 0.1))
 (gr_line (start 115 82) (end 115 88) (layer Edge.Cuts) (width 0.1))
 (gr_line (start 178 80) (end 117 80) (layer Edge.Cuts) (width 0.1))
 (gr_line (start 180 88) (end 180 82) (layer Edge.Cuts) (width 0.1))
 (gr_arc (start 178 88) (end 178 90) (angle -90) (layer Edge.Cuts) (width 0.1))
 (gr_arc (start 117 88) (end 115 88) (angle -90) (layer Edge.Cuts) (width 0.1))
 (gr_arc (start 117 82) (end 117 80) (angle -90) (layer Edge.Cuts) (width 0.1))
 (gr_arc (start 178 82) (end 180 82) (angle -90) (layer Edge.Cuts) (width 0.1)) (via (at 175.25 89) (size 0.8) (layers F.Cu B.Cu) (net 1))
 (segment (start 166.075 82.675) (end 166 82.75) (width 0.2) (layer F.Cu) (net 1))
 (segment (start 163 88) (end 137.5591 88) (width 0.2) (layer B.Cu) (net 2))
 (segment (start 137.5591 88) (end 132.1589 82.5998) (width 0.2) (layer B.Cu) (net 2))
 (via (at 132.1589 82.5998) (size 0.8) (layers F.Cu B.Cu) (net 2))
 (segment (start 129.1502 82.5998) (end 129 82.75) (width 0.2) (layer F.Cu) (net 2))
 (segment (start 132.1589 82.5998) (end 129.1502 82.5998) (width 0.2) (layer F.Cu) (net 2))
 (via (at 149 82.75) (size 0.8) (layers F.Cu B.Cu) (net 3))
 (segment (start 144 82.75) (end 149 82.75) (width 0.2) (layer F.Cu) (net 3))
 (segment (start 149.6483 82.75) (end 149 82.75) (width 0.2) (layer B.Cu) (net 3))
 (segment (start 160.5 82.75) (end 149.6483 82.75) (width 0.2) (layer B.Cu) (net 3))
 (segment (start 165.54 87.79) (end 160.5 82.75) (width 0.2) (layer B.Cu) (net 3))
 (segment (start 165.54 88) (end 165.54 87.79) (width 0.2) (layer B.Cu) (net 3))
 (via (at 162.755 82.675) (size 0.8) (layers F.Cu B.Cu) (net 5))
 (segment (start 162.755 82.675) (end 168.08 88) (width 0.2) (layer B.Cu) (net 5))
 (segment (start 159.075 82.675) (end 159 82.75) (width 0.2) (layer F.Cu) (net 5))
 (segment (start 162.755 82.675) (end 159.075 82.675) (width 0.2) (layer F.Cu) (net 5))
 (segment (start 170.62 88) (end 170.62 86.7497) (width 0.2) (layer B.Cu) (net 4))
 (segment (start 170.62 86.7497) (end 171.2627 86.107) (width 0.2) (layer B.Cu) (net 4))
 (segment (start 171.2627 86.107) (end 171.2627 85.9621) (width 0.2) (layer B.Cu) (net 4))
 (via (at 171.2627 85.9621) (size 0.8) (layers F.Cu B.Cu) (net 4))
 (segment (start 174 83.2248) (end 174 82.75) (width 0.2) (layer F.Cu) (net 4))
 (segment (start 171.2627 85.9621) (end 174 83.2248) (width 0.2) (layer F.Cu) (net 4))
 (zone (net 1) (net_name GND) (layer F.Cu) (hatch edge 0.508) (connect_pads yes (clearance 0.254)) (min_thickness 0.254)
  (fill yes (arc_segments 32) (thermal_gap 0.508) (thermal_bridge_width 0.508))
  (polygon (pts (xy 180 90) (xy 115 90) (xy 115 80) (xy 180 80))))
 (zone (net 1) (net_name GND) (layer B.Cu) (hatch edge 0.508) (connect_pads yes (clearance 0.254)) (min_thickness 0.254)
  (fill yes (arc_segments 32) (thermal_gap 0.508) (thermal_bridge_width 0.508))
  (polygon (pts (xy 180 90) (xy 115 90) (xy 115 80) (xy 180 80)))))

